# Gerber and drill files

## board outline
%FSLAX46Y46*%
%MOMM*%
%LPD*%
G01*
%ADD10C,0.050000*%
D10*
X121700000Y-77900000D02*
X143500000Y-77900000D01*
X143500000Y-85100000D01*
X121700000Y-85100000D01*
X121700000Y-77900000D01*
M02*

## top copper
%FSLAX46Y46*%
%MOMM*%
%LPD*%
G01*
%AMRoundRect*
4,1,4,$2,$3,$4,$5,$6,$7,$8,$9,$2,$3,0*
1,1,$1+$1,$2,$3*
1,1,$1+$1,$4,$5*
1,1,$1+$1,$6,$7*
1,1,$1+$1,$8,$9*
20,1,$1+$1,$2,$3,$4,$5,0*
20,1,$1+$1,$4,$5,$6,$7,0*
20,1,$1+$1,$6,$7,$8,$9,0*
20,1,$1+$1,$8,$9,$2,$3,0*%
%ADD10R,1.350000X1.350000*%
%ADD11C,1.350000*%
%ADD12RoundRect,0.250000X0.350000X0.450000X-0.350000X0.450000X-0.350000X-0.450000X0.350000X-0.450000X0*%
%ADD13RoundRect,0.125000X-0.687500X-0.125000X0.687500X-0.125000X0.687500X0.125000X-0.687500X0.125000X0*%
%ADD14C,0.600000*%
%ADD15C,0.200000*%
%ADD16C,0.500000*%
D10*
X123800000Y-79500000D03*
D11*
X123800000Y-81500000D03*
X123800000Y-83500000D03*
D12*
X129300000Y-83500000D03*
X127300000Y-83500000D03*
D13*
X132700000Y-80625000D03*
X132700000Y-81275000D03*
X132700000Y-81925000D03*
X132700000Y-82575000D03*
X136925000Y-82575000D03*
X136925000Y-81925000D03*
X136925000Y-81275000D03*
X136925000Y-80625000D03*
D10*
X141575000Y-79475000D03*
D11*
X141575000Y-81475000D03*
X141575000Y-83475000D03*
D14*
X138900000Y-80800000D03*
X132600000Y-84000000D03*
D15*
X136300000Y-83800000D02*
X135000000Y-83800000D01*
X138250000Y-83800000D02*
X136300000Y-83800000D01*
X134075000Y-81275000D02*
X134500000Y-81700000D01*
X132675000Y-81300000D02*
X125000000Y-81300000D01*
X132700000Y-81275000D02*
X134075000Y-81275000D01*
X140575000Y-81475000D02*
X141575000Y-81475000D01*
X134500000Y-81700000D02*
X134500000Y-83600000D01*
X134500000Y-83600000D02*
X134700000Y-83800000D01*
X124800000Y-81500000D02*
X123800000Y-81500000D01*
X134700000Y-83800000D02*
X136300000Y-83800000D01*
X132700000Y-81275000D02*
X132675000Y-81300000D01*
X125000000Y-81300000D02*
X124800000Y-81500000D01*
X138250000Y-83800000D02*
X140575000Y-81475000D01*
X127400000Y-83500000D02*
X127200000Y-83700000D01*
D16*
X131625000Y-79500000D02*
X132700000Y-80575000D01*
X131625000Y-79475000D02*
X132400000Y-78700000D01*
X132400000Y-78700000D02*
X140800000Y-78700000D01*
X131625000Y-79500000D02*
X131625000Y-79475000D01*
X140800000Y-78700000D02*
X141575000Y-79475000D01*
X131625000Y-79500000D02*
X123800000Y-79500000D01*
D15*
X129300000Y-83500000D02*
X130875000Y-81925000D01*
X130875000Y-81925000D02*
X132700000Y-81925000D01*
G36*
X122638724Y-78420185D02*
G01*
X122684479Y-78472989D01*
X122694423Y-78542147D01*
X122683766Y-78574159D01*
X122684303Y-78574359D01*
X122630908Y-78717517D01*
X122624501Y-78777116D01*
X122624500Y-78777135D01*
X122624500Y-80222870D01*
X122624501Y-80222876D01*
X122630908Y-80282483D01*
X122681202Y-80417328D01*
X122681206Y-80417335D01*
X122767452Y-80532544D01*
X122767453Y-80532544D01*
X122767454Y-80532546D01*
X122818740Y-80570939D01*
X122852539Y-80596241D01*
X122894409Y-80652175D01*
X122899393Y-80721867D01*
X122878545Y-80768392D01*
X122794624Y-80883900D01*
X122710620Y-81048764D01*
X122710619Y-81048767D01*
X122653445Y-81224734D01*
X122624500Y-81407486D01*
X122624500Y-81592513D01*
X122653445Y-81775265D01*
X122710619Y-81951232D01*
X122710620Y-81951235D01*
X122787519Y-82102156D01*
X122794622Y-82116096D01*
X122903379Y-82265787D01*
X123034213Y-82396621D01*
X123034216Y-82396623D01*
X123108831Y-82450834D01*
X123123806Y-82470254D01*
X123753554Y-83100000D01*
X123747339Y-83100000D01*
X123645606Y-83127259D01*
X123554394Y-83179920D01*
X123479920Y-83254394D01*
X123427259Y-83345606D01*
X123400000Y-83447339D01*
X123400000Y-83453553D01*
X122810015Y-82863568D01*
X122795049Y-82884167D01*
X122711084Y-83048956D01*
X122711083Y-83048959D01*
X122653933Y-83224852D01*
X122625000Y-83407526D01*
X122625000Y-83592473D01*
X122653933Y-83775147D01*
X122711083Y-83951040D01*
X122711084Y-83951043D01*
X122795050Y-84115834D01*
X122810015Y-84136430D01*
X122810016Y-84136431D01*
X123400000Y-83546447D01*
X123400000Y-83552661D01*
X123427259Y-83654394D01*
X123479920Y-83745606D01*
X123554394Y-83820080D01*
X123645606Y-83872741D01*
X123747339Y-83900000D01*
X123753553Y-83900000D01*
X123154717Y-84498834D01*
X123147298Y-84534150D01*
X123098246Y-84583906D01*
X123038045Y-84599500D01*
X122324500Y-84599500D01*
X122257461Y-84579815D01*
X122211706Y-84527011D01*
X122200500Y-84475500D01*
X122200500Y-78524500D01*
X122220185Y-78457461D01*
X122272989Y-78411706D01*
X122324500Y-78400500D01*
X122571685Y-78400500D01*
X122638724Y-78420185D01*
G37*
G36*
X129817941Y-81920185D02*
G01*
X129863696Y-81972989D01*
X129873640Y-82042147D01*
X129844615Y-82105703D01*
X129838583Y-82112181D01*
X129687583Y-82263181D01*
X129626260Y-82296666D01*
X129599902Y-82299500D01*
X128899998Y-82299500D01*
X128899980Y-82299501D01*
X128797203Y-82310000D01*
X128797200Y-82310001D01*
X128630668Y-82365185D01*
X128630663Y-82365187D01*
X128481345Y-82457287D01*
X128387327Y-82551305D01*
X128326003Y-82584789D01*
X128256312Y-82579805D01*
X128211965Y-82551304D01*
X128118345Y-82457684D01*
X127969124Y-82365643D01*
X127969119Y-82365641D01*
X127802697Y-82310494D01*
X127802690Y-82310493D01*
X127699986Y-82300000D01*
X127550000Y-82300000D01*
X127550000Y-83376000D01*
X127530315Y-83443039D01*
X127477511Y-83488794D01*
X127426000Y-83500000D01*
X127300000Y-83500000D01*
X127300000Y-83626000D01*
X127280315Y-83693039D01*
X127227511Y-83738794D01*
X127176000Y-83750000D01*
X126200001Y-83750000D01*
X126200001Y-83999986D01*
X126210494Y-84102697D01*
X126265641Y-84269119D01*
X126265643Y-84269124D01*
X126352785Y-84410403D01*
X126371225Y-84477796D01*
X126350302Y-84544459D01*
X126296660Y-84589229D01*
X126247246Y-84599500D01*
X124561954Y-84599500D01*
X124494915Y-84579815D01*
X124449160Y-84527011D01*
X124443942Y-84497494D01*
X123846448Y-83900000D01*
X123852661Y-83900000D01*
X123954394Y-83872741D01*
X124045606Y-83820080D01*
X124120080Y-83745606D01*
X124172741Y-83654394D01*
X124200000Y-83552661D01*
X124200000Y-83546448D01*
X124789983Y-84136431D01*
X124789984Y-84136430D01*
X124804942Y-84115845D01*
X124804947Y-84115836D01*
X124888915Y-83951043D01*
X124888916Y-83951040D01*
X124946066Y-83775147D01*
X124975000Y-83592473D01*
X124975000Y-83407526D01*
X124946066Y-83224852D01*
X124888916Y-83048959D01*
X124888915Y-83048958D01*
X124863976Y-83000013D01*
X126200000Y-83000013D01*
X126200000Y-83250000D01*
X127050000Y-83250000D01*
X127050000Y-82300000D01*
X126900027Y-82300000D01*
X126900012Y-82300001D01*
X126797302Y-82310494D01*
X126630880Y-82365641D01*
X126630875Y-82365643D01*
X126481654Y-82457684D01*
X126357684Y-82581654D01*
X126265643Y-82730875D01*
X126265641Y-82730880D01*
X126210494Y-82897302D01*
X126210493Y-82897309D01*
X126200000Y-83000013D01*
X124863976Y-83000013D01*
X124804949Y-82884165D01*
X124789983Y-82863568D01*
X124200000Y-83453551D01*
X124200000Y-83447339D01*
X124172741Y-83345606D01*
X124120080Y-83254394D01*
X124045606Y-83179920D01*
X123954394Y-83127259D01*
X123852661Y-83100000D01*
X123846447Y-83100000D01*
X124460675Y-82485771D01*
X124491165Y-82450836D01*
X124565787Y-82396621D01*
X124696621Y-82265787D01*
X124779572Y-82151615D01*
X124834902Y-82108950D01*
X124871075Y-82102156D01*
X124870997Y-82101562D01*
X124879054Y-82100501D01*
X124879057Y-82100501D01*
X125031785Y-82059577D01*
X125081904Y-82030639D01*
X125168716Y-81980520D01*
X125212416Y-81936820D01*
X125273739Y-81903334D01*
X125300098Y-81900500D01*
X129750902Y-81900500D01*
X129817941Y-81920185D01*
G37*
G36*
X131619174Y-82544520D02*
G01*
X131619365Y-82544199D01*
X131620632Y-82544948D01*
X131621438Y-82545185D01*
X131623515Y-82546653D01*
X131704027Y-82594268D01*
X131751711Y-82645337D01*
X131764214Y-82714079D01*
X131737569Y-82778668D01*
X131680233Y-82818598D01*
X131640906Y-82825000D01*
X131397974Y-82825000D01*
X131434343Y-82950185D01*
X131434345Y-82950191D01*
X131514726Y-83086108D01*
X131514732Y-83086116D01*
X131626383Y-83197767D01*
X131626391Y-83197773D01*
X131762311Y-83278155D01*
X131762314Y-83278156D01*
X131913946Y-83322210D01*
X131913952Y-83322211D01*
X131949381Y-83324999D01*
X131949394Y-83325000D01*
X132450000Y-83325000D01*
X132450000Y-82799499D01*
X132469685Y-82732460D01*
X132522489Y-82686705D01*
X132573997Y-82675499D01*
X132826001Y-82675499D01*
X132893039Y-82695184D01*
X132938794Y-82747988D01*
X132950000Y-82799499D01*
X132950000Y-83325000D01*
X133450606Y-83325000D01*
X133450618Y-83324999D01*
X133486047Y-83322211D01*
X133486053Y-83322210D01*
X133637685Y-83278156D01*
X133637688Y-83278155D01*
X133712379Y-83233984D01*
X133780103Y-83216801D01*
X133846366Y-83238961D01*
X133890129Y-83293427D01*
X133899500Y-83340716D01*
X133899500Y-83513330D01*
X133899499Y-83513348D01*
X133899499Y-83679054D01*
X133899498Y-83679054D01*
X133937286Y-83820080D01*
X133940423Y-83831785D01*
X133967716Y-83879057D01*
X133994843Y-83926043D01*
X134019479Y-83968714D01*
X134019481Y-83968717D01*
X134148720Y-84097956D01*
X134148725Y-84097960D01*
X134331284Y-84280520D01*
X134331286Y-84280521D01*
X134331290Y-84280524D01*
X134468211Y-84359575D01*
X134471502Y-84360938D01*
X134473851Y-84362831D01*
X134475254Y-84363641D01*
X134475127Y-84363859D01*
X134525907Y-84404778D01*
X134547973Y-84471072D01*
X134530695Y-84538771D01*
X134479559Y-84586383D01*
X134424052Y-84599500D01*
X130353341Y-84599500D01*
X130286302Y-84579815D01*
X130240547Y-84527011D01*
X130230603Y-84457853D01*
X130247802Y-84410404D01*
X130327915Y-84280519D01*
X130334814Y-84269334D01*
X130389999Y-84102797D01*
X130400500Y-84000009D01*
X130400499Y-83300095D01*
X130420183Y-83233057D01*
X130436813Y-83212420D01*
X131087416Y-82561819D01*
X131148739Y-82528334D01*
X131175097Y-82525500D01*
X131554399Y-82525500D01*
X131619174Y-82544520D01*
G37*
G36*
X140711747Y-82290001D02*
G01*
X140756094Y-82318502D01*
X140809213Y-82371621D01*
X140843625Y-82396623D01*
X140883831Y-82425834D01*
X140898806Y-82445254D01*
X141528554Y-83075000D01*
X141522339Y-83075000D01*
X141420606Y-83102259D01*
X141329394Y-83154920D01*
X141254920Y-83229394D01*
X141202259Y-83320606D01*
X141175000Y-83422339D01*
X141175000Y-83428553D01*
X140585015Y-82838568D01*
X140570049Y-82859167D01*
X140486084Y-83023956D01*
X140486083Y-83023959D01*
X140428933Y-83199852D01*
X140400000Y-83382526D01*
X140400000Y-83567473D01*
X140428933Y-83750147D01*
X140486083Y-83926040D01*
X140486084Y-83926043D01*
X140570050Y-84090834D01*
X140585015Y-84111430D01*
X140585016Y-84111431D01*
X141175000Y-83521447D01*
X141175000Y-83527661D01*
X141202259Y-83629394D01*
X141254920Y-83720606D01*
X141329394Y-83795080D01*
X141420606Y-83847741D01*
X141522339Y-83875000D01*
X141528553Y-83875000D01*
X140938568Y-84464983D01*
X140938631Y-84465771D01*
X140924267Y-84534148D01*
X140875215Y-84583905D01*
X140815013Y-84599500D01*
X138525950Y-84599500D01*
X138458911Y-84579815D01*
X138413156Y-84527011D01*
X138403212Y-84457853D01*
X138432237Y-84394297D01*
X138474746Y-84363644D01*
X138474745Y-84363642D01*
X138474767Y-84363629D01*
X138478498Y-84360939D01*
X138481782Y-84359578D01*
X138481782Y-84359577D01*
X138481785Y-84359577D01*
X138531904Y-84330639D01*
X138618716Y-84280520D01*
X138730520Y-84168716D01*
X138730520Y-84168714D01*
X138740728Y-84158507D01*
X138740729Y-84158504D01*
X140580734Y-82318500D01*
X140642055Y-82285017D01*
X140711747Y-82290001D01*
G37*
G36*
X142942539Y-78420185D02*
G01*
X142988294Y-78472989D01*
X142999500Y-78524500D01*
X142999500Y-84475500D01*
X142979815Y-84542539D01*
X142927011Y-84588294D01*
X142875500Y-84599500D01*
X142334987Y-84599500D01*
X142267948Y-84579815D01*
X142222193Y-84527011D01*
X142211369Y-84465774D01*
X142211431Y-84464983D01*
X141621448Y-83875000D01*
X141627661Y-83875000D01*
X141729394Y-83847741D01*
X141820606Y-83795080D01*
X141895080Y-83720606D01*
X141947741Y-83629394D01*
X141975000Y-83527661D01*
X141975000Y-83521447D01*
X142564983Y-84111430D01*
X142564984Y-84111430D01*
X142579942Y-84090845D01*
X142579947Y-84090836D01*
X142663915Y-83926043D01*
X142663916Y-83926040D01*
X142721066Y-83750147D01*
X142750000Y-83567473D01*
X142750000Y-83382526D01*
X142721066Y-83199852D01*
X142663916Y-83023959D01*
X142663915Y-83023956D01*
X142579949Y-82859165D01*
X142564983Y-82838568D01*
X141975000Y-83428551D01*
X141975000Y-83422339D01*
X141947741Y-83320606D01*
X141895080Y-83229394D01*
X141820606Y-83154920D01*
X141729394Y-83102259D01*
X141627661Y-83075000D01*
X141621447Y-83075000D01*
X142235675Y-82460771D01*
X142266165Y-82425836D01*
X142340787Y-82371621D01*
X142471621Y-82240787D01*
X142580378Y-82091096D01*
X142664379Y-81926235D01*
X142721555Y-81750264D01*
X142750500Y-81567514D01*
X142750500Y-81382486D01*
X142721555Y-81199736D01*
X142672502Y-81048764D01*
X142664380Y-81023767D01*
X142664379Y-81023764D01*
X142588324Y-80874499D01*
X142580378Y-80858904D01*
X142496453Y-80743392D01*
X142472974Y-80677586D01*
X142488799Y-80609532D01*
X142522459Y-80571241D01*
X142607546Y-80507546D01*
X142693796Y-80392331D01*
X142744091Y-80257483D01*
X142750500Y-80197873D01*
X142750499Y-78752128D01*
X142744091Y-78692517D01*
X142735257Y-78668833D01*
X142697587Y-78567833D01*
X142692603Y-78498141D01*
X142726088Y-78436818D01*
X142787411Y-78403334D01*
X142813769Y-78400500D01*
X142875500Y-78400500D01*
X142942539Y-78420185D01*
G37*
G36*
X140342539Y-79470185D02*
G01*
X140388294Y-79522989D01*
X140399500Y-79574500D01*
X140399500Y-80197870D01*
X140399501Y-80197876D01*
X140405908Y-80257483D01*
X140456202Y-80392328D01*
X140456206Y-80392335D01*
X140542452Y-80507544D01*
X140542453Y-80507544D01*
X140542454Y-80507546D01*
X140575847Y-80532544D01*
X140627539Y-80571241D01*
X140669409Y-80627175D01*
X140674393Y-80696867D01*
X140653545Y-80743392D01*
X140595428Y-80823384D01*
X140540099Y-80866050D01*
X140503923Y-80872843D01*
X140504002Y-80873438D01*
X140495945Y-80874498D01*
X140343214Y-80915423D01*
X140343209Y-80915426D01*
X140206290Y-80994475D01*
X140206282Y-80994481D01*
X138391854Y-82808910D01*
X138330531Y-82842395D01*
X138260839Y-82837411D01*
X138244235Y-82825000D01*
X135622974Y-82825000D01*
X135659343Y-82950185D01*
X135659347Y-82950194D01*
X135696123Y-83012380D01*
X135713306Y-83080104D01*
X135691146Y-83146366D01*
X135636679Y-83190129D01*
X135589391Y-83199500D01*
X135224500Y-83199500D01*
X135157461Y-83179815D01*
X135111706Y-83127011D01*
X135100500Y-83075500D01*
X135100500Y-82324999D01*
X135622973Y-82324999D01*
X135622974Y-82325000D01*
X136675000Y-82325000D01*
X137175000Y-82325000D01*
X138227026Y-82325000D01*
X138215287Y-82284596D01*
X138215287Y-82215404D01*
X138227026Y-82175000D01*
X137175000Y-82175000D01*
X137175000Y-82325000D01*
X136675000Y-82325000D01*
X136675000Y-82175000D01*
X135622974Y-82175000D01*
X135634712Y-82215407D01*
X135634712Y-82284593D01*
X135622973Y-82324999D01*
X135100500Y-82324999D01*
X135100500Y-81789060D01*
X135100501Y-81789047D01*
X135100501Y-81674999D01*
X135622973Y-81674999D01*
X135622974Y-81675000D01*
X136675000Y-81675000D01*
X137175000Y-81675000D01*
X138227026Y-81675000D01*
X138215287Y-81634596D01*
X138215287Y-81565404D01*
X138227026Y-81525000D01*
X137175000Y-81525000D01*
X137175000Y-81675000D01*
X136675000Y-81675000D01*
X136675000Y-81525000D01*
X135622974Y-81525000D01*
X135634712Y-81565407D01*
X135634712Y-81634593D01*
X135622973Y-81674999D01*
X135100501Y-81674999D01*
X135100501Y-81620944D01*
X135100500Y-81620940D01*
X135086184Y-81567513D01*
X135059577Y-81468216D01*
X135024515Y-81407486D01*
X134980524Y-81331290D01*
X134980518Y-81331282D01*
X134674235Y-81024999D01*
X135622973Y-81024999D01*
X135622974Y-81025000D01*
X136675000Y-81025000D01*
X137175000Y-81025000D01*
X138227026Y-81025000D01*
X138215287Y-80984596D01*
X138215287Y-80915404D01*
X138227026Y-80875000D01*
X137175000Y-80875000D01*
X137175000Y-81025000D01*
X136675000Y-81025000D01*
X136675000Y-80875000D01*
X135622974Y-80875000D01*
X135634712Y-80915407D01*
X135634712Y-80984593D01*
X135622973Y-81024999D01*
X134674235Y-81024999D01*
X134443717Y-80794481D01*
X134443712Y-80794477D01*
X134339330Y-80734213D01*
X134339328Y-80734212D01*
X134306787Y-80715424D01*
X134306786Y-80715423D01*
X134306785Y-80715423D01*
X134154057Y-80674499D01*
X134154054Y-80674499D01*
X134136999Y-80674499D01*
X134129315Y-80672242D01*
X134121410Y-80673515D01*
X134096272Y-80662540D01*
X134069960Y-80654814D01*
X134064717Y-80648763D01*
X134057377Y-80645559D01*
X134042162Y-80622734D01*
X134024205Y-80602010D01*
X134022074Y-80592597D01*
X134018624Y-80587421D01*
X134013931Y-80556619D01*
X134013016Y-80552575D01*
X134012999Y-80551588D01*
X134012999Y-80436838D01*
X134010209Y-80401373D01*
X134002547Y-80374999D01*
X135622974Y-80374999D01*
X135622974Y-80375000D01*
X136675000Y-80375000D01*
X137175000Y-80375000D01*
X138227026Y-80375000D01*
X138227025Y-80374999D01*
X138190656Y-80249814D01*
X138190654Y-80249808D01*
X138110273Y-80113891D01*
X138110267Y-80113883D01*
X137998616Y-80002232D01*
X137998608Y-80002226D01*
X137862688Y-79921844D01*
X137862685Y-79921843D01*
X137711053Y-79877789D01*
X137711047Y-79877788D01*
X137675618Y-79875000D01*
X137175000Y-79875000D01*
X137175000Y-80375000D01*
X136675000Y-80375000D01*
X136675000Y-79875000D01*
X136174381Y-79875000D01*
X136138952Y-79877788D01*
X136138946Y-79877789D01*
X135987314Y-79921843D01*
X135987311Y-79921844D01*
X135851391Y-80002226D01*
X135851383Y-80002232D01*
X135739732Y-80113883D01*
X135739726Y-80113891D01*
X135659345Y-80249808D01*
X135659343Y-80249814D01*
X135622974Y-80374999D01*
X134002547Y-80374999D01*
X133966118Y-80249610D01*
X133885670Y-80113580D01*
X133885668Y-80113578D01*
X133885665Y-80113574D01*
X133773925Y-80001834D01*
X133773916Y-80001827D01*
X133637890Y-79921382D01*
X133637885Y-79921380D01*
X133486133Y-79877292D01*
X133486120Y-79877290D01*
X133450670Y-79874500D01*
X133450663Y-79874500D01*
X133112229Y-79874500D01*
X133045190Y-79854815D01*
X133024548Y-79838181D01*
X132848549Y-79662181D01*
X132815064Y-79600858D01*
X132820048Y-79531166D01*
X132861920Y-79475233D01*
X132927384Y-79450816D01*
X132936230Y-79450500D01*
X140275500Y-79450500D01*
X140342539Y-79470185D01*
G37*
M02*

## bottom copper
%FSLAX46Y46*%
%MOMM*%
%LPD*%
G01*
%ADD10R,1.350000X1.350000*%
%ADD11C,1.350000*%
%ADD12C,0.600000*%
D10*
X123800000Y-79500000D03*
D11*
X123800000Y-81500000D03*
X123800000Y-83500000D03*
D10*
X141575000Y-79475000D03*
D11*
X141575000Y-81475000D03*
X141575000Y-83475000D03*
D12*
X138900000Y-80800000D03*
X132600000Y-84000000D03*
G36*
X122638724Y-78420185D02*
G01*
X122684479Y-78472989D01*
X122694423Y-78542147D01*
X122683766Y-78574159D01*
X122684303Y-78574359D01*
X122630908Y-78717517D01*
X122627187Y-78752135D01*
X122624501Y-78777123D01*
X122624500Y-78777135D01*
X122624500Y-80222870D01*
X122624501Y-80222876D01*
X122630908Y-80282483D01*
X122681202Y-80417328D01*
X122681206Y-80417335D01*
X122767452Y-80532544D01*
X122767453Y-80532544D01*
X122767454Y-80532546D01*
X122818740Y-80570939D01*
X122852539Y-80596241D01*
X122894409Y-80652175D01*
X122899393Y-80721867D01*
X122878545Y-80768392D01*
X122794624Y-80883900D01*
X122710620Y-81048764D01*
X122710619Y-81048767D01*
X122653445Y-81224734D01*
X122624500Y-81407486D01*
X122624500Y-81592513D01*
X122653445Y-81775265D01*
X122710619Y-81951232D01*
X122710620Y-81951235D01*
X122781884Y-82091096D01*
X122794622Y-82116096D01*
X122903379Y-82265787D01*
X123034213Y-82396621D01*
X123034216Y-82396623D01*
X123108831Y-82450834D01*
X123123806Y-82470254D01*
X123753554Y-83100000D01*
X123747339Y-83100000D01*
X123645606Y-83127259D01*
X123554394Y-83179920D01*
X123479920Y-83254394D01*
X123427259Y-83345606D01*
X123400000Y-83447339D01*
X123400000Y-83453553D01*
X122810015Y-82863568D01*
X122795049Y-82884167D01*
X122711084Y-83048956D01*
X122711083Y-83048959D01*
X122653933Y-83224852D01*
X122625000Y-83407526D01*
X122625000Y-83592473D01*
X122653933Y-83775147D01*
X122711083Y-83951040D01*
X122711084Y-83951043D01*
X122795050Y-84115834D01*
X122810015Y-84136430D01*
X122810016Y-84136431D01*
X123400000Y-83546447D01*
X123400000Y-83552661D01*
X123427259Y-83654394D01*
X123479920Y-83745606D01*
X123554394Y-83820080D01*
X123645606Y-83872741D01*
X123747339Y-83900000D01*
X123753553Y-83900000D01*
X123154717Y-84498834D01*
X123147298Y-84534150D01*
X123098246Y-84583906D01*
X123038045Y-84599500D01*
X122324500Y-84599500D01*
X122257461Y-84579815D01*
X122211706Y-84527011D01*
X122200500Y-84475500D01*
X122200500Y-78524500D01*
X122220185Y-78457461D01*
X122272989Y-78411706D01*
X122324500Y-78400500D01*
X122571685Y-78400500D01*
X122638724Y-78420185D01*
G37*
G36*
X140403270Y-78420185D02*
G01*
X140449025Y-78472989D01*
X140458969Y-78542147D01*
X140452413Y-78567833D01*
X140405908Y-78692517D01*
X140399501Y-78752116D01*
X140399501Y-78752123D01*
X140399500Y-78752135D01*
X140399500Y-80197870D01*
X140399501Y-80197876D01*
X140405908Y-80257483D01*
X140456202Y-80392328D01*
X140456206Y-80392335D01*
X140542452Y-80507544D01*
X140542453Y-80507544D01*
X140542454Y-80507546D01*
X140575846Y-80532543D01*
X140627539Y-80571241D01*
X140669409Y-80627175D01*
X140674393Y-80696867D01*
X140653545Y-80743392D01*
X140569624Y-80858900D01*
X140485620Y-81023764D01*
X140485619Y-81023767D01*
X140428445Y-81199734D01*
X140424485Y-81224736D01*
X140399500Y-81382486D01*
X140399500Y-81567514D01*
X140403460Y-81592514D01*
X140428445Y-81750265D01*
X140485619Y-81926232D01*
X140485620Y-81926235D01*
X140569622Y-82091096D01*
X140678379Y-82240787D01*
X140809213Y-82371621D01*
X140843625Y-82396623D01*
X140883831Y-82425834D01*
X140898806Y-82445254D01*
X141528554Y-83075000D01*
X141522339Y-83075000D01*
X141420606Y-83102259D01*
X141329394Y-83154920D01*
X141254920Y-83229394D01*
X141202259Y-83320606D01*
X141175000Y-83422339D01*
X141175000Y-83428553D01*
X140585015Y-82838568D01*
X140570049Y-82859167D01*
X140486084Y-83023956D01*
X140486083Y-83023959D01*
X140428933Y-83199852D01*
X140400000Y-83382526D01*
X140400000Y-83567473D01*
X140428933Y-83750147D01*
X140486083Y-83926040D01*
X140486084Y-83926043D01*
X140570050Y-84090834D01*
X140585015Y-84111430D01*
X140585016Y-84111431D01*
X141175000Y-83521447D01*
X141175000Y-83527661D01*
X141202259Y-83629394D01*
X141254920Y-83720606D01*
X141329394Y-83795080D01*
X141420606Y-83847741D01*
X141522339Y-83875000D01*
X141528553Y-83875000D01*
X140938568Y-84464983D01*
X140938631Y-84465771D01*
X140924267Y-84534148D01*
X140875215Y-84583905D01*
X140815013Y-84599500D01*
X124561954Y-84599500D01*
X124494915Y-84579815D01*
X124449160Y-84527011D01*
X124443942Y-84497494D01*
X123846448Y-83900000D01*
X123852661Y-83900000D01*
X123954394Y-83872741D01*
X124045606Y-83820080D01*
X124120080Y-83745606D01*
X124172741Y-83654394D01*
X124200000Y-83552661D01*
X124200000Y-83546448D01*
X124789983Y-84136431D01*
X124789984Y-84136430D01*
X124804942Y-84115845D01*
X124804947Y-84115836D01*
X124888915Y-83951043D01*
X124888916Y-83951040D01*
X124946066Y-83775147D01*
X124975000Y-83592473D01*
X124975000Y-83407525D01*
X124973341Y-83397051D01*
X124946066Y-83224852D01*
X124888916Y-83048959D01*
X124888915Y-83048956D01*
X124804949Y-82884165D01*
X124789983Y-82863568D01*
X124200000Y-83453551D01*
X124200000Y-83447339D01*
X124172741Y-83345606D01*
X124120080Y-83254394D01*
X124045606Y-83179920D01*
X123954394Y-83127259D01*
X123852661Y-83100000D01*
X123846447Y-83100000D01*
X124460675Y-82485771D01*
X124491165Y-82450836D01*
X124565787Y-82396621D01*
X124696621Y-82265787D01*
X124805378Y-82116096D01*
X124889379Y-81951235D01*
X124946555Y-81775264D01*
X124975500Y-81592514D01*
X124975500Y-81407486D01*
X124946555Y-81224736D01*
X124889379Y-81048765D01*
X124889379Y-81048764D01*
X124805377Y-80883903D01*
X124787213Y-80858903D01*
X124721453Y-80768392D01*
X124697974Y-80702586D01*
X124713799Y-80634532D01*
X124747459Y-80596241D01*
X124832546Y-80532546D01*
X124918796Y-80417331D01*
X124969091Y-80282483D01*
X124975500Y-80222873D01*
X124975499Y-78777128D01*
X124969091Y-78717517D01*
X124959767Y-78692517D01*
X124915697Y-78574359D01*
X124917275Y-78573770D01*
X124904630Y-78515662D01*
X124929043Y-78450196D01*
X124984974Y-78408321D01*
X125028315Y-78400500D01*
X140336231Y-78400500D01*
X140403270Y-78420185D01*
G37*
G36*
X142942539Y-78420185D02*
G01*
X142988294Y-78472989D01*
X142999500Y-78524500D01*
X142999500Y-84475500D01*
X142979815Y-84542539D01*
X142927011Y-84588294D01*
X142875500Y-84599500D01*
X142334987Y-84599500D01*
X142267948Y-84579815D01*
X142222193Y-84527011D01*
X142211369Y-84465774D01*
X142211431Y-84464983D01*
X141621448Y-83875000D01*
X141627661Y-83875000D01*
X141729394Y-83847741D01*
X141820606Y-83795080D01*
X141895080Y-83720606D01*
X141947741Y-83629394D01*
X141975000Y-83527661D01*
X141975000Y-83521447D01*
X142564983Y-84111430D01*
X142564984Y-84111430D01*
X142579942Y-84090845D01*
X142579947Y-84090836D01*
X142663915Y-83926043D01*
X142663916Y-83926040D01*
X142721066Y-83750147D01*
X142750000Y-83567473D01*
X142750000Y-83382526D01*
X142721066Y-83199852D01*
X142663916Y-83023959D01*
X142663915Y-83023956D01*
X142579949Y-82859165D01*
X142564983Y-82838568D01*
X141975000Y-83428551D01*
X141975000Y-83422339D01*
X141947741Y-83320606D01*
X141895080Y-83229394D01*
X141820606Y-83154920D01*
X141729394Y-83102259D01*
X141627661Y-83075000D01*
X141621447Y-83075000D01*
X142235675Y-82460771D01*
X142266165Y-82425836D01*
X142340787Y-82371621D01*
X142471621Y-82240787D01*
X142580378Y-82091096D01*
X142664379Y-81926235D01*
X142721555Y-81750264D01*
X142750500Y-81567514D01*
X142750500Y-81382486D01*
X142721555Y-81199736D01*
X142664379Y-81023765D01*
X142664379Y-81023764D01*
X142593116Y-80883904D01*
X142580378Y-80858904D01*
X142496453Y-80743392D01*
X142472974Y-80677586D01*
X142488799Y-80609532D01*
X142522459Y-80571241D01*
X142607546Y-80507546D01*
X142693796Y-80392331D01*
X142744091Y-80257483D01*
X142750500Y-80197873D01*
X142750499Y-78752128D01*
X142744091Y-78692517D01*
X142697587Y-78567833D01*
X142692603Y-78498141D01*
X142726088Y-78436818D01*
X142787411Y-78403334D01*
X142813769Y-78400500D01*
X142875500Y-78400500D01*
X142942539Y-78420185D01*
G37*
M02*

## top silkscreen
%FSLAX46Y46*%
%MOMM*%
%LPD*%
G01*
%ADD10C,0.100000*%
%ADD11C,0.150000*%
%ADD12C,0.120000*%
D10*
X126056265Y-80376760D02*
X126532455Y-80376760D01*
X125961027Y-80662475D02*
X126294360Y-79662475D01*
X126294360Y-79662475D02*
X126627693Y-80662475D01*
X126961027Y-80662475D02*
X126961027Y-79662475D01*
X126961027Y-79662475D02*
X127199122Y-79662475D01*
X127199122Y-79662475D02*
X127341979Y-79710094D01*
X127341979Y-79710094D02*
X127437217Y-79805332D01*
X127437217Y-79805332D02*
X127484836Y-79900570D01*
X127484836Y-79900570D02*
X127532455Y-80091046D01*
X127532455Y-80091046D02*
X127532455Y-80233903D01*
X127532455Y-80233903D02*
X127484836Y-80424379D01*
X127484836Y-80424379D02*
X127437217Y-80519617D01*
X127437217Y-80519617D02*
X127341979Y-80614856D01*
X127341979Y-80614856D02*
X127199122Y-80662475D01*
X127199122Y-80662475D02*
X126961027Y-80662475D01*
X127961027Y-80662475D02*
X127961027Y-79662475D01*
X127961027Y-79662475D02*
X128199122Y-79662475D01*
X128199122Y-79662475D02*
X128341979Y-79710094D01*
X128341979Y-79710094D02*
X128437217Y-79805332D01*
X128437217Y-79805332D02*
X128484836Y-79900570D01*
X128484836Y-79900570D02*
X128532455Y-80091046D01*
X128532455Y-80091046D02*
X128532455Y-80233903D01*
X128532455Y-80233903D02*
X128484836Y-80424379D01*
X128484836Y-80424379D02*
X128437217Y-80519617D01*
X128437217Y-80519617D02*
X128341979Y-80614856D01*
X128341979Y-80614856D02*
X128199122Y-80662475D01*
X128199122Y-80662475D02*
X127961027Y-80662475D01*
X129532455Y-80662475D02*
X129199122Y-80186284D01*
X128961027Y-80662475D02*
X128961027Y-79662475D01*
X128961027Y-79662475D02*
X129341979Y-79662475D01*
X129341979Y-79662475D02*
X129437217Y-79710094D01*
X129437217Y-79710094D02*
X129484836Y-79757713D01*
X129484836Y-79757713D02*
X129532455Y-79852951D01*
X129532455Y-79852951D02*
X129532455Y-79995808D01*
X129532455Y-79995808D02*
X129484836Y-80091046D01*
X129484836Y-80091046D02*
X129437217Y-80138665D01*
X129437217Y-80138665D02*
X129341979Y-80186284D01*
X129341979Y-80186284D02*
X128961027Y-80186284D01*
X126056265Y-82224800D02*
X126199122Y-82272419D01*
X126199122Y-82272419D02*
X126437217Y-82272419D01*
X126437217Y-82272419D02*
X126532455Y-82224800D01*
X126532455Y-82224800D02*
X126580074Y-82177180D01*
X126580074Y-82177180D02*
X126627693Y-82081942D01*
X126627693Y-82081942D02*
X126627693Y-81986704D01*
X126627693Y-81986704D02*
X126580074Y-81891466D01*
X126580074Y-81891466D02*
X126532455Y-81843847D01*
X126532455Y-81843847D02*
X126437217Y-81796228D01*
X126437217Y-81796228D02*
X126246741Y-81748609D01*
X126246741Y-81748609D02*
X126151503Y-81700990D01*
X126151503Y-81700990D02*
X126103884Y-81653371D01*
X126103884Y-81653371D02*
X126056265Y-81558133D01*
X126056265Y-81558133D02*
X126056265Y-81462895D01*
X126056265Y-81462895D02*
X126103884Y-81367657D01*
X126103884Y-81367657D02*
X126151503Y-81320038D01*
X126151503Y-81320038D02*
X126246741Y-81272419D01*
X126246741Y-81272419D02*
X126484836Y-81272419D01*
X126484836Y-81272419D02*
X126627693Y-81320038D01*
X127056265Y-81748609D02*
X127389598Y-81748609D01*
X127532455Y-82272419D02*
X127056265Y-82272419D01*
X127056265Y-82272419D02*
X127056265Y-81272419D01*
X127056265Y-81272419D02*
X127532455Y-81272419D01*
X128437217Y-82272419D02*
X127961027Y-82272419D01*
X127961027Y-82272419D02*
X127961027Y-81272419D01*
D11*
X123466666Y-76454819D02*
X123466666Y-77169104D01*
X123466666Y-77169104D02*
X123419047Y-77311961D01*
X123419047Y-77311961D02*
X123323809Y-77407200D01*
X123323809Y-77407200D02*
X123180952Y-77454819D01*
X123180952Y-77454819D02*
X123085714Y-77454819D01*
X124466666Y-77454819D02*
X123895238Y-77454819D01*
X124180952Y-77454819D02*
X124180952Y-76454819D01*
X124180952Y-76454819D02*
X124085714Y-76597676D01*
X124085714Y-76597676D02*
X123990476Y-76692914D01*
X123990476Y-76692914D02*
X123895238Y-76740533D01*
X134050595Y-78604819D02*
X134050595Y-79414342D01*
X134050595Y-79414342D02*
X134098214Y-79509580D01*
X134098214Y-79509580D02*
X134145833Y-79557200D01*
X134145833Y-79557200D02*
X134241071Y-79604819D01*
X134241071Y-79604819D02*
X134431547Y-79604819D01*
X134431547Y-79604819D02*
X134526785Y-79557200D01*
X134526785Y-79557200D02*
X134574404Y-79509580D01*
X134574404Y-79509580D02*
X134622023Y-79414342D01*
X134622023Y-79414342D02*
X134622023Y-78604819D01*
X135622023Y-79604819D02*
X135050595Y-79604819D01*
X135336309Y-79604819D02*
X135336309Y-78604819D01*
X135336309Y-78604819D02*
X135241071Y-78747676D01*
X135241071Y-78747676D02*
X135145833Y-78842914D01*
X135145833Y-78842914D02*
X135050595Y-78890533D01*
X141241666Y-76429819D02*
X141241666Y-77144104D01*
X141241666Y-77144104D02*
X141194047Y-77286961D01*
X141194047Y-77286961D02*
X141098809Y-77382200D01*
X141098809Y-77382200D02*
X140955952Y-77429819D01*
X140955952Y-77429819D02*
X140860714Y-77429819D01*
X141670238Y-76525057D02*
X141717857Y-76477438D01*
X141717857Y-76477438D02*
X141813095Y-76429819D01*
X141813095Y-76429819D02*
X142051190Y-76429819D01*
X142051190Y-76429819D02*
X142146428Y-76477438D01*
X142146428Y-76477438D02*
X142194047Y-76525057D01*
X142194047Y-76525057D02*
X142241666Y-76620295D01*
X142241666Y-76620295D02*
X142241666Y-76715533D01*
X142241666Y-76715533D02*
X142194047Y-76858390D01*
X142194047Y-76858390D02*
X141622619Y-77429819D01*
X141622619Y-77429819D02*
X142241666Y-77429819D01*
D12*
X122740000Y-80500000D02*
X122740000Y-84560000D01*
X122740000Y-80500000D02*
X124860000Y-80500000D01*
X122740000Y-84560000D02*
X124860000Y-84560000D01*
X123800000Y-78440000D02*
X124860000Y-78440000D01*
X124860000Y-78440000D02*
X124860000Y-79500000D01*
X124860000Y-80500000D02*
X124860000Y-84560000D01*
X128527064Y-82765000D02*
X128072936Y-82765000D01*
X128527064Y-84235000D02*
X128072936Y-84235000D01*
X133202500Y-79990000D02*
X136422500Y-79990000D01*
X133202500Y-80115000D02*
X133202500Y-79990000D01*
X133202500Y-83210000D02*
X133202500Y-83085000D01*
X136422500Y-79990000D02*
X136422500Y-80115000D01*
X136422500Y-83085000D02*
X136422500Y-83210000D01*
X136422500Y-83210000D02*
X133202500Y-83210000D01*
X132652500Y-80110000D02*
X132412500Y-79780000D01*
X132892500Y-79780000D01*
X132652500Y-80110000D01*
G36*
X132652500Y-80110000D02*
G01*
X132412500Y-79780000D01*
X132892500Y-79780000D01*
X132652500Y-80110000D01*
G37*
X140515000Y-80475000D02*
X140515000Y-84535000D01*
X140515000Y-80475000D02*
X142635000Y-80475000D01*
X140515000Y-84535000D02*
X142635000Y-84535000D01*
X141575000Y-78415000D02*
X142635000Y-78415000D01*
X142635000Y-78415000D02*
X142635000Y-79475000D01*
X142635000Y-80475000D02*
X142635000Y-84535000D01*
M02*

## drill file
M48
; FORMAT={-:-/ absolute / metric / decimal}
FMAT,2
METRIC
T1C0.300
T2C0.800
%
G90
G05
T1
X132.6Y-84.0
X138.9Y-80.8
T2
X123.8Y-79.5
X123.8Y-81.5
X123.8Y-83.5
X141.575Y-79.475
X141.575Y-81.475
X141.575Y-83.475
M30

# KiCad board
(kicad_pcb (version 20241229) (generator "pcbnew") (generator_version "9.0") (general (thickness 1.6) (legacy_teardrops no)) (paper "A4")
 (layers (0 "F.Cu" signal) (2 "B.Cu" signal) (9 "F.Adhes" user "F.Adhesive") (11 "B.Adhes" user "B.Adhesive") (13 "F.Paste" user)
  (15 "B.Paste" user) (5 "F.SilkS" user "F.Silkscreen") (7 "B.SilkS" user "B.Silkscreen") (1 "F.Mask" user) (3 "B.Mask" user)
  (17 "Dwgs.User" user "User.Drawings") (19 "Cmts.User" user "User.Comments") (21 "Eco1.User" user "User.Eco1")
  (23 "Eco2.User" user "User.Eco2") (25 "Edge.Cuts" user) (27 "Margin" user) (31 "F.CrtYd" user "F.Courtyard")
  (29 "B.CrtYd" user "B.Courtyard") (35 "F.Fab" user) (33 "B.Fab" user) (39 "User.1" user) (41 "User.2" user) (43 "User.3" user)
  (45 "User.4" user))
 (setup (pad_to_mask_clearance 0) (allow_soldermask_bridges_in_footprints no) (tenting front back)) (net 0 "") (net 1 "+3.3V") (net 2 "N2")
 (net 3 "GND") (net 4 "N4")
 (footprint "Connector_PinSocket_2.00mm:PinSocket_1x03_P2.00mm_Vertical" (layer "F.Cu") (at 123.8 79.5)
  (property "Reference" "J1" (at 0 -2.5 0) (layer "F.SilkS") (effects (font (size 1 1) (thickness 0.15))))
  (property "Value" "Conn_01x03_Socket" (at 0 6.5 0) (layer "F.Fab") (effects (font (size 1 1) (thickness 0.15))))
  (fp_line (start -1.06 1) (end -1.06 5.06) (stroke (width 0.12) (type solid)) (layer "F.SilkS"))
  (fp_line (start -1.06 1) (end 1.06 1) (stroke (width 0.12) (type solid)) (layer "F.SilkS"))
  (fp_line (start -1.06 5.06) (end 1.06 5.06) (stroke (width 0.12) (type solid)) (layer "F.SilkS"))
  (fp_line (start 0 -1.06) (end 1.06 -1.06) (stroke (width 0.12) (type solid)) (layer "F.SilkS"))
  (fp_line (start 1.06 -1.06) (end 1.06 0) (stroke (width 0.12) (type solid)) (layer "F.SilkS"))
  (fp_line (start 1.06 1) (end 1.06 5.06) (stroke (width 0.12) (type solid)) (layer "F.SilkS"))
  (pad "1" thru_hole rect (at 0 0) (size 1.35 1.35) (drill 0.8) (layers "*.Cu" "*.Mask") (remove_unused_layers no) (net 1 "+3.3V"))
  (pad "2" thru_hole circle (at 0 2) (size 1.35 1.35) (drill 0.8) (layers "*.Cu" "*.Mask") (remove_unused_layers no) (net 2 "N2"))
  (pad "3" thru_hole circle (at 0 4) (size 1.35 1.35) (drill 0.8) (layers "*.Cu" "*.Mask") (remove_unused_layers no) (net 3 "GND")))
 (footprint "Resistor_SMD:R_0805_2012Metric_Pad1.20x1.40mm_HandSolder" (layer "F.Cu") (at 128.3 83.5 180)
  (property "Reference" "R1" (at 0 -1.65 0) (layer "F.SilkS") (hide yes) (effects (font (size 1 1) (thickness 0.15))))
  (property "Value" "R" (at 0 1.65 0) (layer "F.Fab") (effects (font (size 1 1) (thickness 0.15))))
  (fp_line (start -0.227064 0.735) (end 0.227064 0.735) (stroke (width 0.12) (type solid)) (layer "F.SilkS"))
  (fp_line (start -0.227064 -0.735) (end 0.227064 -0.735) (stroke (width 0.12) (type solid)) (layer "F.SilkS"))
  (pad "1" smd roundrect (at -1 0 180) (size 1.2 1.4) (layers "F.Cu" "F.Mask" "F.Paste") (roundrect_rratio 0.208333) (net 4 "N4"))
  (pad "2" smd roundrect (at 1 0 180) (size 1.2 1.4) (layers "F.Cu" "F.Mask" "F.Paste") (roundrect_rratio 0.208333) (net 3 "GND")))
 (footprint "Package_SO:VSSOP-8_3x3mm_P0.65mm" (layer "F.Cu") (at 134.8125 81.6)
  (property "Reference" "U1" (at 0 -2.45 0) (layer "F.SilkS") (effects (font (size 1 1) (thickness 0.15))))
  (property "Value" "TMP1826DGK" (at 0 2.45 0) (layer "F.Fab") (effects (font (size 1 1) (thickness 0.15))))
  (fp_line (start -1.61 -1.61) (end 1.61 -1.61) (stroke (width 0.12) (type solid)) (layer "F.SilkS"))
  (fp_line (start -1.61 -1.485) (end -1.61 -1.61) (stroke (width 0.12) (type solid)) (layer "F.SilkS"))
  (fp_line (start -1.61 1.61) (end -1.61 1.485) (stroke (width 0.12) (type solid)) (layer "F.SilkS"))
  (fp_line (start 1.61 -1.61) (end 1.61 -1.485) (stroke (width 0.12) (type solid)) (layer "F.SilkS"))
  (fp_line (start 1.61 1.485) (end 1.61 1.61) (stroke (width 0.12) (type solid)) (layer "F.SilkS"))
  (fp_line (start 1.61 1.61) (end -1.61 1.61) (stroke (width 0.12) (type solid)) (layer "F.SilkS"))
  (fp_poly (pts (xy -2.16 -1.49) (xy -2.4 -1.82) (xy -1.92 -1.82)) (stroke (width 0.12) (type solid)) (fill yes) (layer "F.SilkS"))
  (pad "1" smd roundrect (at -2.1125 -0.975) (size 1.625 0.5) (layers "F.Cu" "F.Mask" "F.Paste") (roundrect_rratio 0.25) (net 1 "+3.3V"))
  (pad "2" smd roundrect (at -2.1125 -0.325) (size 1.625 0.5) (layers "F.Cu" "F.Mask" "F.Paste") (roundrect_rratio 0.25) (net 2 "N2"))
  (pad "3" smd roundrect (at -2.1125 0.325) (size 1.625 0.5) (layers "F.Cu" "F.Mask" "F.Paste") (roundrect_rratio 0.25) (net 4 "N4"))
  (pad "4" smd roundrect (at -2.1125 0.975) (size 1.625 0.5) (layers "F.Cu" "F.Mask" "F.Paste") (roundrect_rratio 0.25) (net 3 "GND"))
  (pad "5" smd roundrect (at 2.1125 0.975) (size 1.625 0.5) (layers "F.Cu" "F.Mask" "F.Paste") (roundrect_rratio 0.25) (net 3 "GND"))
  (pad "6" smd roundrect (at 2.1125 0.325) (size 1.625 0.5) (layers "F.Cu" "F.Mask" "F.Paste") (roundrect_rratio 0.25) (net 3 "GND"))
  (pad "7" smd roundrect (at 2.1125 -0.325) (size 1.625 0.5) (layers "F.Cu" "F.Mask" "F.Paste") (roundrect_rratio 0.25) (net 3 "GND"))
  (pad "8" smd roundrect (at 2.1125 -0.975) (size 1.625 0.5) (layers "F.Cu" "F.Mask" "F.Paste") (roundrect_rratio 0.25) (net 3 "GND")))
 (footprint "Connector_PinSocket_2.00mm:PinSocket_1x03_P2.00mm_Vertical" (layer "F.Cu") (at 141.575 79.475)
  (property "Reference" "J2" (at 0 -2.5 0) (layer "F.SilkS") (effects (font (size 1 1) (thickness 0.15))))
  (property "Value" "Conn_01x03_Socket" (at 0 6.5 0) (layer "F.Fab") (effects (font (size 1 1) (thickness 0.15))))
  (fp_line (start -1.06 1) (end -1.06 5.06) (stroke (width 0.12) (type solid)) (layer "F.SilkS"))
  (fp_line (start -1.06 1) (end 1.06 1) (stroke (width 0.12) (type solid)) (layer "F.SilkS"))
  (fp_line (start -1.06 5.06) (end 1.06 5.06) (stroke (width 0.12) (type solid)) (layer "F.SilkS"))
  (fp_line (start 0 -1.06) (end 1.06 -1.06) (stroke (width 0.12) (type solid)) (layer "F.SilkS"))
  (fp_line (start 1.06 -1.06) (end 1.06 0) (stroke (width 0.12) (type solid)) (layer "F.SilkS"))
  (fp_line (start 1.06 1) (end 1.06 5.06) (stroke (width 0.12) (type solid)) (layer "F.SilkS"))
  (pad "1" thru_hole rect (at 0 0) (size 1.35 1.35) (drill 0.8) (layers "*.Cu" "*.Mask") (remove_unused_layers no) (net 1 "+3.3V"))
  (pad "2" thru_hole circle (at 0 2) (size 1.35 1.35) (drill 0.8) (layers "*.Cu" "*.Mask") (remove_unused_layers no) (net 2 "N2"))
  (pad "3" thru_hole circle (at 0 4) (size 1.35 1.35) (drill 0.8) (layers "*.Cu" "*.Mask") (remove_unused_layers no) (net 3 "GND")))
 (gr_rect (start 121.7 77.9) (end 143.5 85.1) (stroke (width 0.05) (type default)) (fill no) (layer "Edge.Cuts"))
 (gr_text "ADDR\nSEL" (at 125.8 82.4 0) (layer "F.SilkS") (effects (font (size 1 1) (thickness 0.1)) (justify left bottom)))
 (segment (start 136.3 83.8) (end 135 83.8) (width 0.2) (layer "F.Cu") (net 2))
 (segment (start 138.25 83.8) (end 136.3 83.8) (width 0.2) (layer "F.Cu") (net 2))
 (segment (start 134.075 81.275) (end 134.5 81.7) (width 0.2) (layer "F.Cu") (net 2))
 (segment (start 132.675 81.3) (end 125 81.3) (width 0.2) (layer "F.Cu") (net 2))
 (segment (start 132.7 81.275) (end 134.075 81.275) (width 0.2) (layer "F.Cu") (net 2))
 (segment (start 140.575 81.475) (end 141.575 81.475) (width 0.2) (layer "F.Cu") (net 2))
 (segment (start 134.5 81.7) (end 134.5 83.6) (width 0.2) (layer "F.Cu") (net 2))
 (segment (start 134.5 83.6) (end 134.7 83.8) (width 0.2) (layer "F.Cu") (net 2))
 (segment (start 124.8 81.5) (end 123.8 81.5) (width 0.2) (layer "F.Cu") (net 2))
 (segment (start 134.7 83.8) (end 136.3 83.8) (width 0.2) (layer "F.Cu") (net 2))
 (segment (start 132.7 81.275) (end 132.675 81.3) (width 0.2) (layer "F.Cu") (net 2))
 (segment (start 125 81.3) (end 124.8 81.5) (width 0.2) (layer "F.Cu") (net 2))
 (segment (start 138.25 83.8) (end 140.575 81.475) (width 0.2) (layer "F.Cu") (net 2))
 (segment (start 127.4 83.5) (end 127.2 83.7) (width 0.2) (layer "F.Cu") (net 3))
 (via (at 138.9 80.8) (size 0.6) (drill 0.3) (layers "F.Cu" "B.Cu") (free yes) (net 3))
 (via (at 132.6 84) (size 0.6) (drill 0.3) (layers "F.Cu" "B.Cu") (free yes) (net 3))
 (segment (start 131.625 79.5) (end 132.7 80.575) (width 0.5) (layer "F.Cu") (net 1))
 (segment (start 131.625 79.475) (end 132.4 78.7) (width 0.5) (layer "F.Cu") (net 1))
 (segment (start 132.4 78.7) (end 140.8 78.7) (width 0.5) (layer "F.Cu") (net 1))
 (segment (start 131.625 79.5) (end 131.625 79.475) (width 0.5) (layer "F.Cu") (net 1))
 (segment (start 140.8 78.7) (end 141.575 79.475) (width 0.5) (layer "F.Cu") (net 1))
 (segment (start 131.625 79.5) (end 123.8 79.5) (width 0.5) (layer "F.Cu") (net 1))
 (segment (start 129.3 83.5) (end 130.875 81.925) (width 0.2) (layer "F.Cu") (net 4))
 (segment (start 130.875 81.925) (end 132.7 81.925) (width 0.2) (layer "F.Cu") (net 4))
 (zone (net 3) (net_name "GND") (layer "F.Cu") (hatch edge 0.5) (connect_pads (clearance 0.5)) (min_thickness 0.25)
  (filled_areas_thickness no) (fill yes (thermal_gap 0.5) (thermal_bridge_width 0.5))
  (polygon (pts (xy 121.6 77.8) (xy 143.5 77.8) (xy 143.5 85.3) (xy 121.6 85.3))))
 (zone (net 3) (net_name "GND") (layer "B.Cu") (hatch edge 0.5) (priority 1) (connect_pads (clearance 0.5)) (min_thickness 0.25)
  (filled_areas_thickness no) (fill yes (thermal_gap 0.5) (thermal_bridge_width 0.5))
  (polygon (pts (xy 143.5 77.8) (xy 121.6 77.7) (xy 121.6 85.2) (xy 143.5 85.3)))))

